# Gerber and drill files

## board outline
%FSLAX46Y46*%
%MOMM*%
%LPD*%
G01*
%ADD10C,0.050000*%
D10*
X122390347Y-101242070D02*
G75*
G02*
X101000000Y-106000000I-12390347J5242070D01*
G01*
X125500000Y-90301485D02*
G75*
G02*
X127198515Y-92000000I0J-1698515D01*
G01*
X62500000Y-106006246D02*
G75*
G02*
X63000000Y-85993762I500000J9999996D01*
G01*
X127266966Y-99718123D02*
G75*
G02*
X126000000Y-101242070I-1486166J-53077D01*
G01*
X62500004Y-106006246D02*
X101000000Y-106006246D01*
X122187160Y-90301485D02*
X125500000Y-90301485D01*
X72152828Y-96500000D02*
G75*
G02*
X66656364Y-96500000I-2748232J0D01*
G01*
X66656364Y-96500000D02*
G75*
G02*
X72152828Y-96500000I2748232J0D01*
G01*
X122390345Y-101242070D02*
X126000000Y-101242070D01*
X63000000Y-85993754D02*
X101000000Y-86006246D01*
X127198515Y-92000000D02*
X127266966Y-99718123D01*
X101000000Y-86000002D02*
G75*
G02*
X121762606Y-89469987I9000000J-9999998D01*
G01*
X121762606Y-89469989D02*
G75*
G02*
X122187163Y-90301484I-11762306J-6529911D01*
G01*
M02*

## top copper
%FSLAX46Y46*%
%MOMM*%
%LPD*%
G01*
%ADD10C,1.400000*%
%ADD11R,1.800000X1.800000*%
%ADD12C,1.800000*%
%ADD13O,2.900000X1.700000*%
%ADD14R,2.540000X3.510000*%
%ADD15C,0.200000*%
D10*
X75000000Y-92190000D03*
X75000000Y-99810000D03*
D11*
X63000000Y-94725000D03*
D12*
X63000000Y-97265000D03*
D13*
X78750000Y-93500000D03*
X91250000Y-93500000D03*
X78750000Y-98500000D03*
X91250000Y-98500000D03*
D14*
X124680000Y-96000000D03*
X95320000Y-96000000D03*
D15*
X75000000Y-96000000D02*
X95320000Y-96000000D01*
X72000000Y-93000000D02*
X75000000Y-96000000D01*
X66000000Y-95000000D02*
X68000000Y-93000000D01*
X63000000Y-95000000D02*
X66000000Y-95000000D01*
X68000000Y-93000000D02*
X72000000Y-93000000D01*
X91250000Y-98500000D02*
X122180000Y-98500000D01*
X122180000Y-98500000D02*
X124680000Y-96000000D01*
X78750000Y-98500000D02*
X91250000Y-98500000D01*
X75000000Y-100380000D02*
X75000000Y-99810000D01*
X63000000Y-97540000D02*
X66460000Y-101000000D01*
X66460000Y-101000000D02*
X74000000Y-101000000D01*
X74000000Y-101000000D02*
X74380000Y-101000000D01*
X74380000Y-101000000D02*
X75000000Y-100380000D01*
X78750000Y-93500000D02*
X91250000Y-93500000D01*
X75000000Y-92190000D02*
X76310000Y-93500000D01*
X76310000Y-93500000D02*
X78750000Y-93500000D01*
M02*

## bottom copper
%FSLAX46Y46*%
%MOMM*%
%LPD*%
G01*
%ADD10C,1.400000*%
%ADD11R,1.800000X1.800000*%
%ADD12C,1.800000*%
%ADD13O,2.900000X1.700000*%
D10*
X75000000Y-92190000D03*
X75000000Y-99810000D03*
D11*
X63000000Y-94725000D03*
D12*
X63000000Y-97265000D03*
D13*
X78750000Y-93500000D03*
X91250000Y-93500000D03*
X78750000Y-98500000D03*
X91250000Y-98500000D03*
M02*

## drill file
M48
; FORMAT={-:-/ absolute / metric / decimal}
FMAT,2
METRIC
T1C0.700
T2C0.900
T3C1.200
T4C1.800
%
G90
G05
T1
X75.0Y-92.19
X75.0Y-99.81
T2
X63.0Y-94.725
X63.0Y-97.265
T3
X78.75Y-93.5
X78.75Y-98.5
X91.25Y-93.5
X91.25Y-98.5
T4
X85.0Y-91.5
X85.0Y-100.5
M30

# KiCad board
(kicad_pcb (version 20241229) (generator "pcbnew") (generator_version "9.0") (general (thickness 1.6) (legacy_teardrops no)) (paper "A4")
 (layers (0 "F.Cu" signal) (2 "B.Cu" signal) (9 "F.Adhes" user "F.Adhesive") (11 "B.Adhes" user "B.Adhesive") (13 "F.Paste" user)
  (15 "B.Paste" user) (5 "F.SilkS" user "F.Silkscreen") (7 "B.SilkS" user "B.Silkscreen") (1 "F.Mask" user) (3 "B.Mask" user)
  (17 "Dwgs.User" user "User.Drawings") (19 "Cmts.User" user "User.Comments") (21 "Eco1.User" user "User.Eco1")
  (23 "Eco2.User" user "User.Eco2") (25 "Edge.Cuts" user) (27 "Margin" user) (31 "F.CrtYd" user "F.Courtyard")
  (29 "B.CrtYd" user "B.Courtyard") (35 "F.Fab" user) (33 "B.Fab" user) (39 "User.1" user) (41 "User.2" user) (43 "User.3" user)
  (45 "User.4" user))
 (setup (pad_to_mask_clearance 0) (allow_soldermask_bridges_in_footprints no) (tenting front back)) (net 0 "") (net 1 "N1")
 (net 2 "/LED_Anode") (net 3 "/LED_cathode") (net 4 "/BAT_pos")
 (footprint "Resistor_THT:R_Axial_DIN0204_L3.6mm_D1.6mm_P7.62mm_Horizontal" (layer "F.Cu") (at 75 92.19 -90)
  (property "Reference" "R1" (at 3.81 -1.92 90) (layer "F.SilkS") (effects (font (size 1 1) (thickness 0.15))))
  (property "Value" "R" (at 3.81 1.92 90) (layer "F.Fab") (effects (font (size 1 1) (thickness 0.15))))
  (pad "1" thru_hole circle (at 0 0 270) (size 1.4 1.4) (drill 0.7) (layers "*.Cu" "*.Mask") (remove_unused_layers no) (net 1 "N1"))
  (pad "2" thru_hole circle (at 7.62 0 270) (size 1.4 1.4) (drill 0.7) (layers "*.Cu" "*.Mask") (remove_unused_layers no)
   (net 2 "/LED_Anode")))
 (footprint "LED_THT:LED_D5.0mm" (layer "F.Cu") (at 63 94.725 -90)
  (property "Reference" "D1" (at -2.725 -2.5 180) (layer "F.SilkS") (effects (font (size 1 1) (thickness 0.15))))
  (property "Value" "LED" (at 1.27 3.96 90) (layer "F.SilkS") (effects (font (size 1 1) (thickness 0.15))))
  (pad "1" thru_hole rect (at 0 0 270) (size 1.8 1.8) (drill 0.9) (layers "*.Cu" "*.Mask") (remove_unused_layers no) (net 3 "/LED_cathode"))
  (pad "2" thru_hole circle (at 2.54 0 270) (size 1.8 1.8) (drill 0.9) (layers "*.Cu" "*.Mask") (remove_unused_layers no)
   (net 2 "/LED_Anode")))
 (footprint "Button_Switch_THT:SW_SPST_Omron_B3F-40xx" (layer "F.Cu") (at 78.75 93.5)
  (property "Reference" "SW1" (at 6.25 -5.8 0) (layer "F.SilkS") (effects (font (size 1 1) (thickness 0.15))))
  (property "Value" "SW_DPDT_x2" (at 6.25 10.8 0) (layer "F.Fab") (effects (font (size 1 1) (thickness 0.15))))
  (pad "" np_thru_hole circle (at 6.25 -2) (size 1.8 1.8) (drill 1.8) (layers "*.Cu" "*.Mask"))
  (pad "" np_thru_hole circle (at 6.25 7) (size 1.8 1.8) (drill 1.8) (layers "*.Cu" "*.Mask"))
  (pad "1" thru_hole oval (at 0 0) (size 2.9 1.7) (drill 1.2) (layers "*.Cu" "*.Mask") (remove_unused_layers no) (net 1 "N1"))
  (pad "1" thru_hole oval (at 12.5 0) (size 2.9 1.7) (drill 1.2) (layers "*.Cu" "*.Mask") (remove_unused_layers no) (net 1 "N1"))
  (pad "2" thru_hole oval (at 0 5) (size 2.9 1.7) (drill 1.2) (layers "*.Cu" "*.Mask") (remove_unused_layers no) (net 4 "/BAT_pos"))
  (pad "2" thru_hole oval (at 12.5 5) (size 2.9 1.7) (drill 1.2) (layers "*.Cu" "*.Mask") (remove_unused_layers no) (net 4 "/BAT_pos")))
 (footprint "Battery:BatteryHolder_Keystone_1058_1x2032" (layer "F.Cu") (at 110 96 180)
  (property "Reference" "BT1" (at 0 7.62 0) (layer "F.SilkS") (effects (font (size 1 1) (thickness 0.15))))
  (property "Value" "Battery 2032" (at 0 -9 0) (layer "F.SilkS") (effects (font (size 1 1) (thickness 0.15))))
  (pad "1" smd rect (at -14.68 0 180) (size 2.54 3.51) (layers "F.Cu" "F.Mask" "F.Paste") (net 4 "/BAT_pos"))
  (pad "2" smd rect (at 14.68 0 180) (size 2.54 3.51) (layers "F.Cu" "F.Mask" "F.Paste") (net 3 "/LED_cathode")))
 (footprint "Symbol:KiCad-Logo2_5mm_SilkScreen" (layer "B.Cu") (at 110 94.5 180)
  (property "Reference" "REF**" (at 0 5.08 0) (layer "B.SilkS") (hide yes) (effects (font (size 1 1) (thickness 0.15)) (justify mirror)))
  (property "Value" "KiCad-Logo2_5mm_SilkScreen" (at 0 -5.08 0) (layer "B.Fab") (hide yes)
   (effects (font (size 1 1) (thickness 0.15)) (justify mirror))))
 (gr_arc (start 122.390347 101.24207) (mid 112.921145 109.132666) (end 101 106) (stroke (width 0.05) (type default)) (locked yes)
  (layer "Edge.Cuts"))
 (gr_arc (start 125.5 90.301485) (mid 126.701031 90.798969) (end 127.198515 92) (stroke (width 0.05) (type default)) (locked yes)
  (layer "Edge.Cuts"))
 (gr_arc (start 62.5 106.006246) (mid 52.990631 95.756168) (end 63 85.993754) (stroke (width 0.05) (type default)) (locked yes)
  (layer "Edge.Cuts"))
 (gr_arc (start 127.266966 99.718123) (mid 126.924335 100.721902) (end 126 101.24207) (stroke (width 0.05) (type default)) (locked yes)
  (layer "Edge.Cuts"))
 (gr_line (start 62.500004 106.006246) (end 101 106.006246) (stroke (width 0.05) (type default)) (locked yes) (layer "Edge.Cuts"))
 (gr_line (start 122.18716 90.301485) (end 125.5 90.301485) (stroke (width 0.05) (type solid)) (locked yes) (layer "Edge.Cuts"))
 (gr_circle (center 69.404596 96.5) (end 71.707372 98) (stroke (width 0.05) (type default)) (fill no) (layer "Edge.Cuts"))
 (gr_line (start 122.390345 101.24207) (end 126 101.24207) (stroke (width 0.05) (type default)) (locked yes) (layer "Edge.Cuts"))
 (gr_line (start 63 85.993754) (end 101 86.006246) (stroke (width 0.05) (type default)) (locked yes) (layer "Edge.Cuts"))
 (gr_line (start 127.198515 92) (end 127.266966 99.718123) (stroke (width 0.05) (type default)) (locked yes) (layer "Edge.Cuts"))
 (gr_arc (start 101 86.000002) (mid 112.217701 82.73042) (end 121.762606 89.469987) (stroke (width 0.05) (type default)) (locked yes)
  (layer "Edge.Cuts"))
 (gr_arc (start 121.762606 89.469989) (mid 121.982098 89.882053) (end 122.18716 90.301485) (stroke (width 0.05) (type default)) (locked yes)
  (layer "Edge.Cuts"))
 (segment (start 75 96) (end 95.32 96) (width 0.2) (layer "F.Cu") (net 3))
 (segment (start 72 93) (end 75 96) (width 0.2) (layer "F.Cu") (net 3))
 (segment (start 66 95) (end 68 93) (width 0.2) (layer "F.Cu") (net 3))
 (segment (start 63 95) (end 66 95) (width 0.2) (layer "F.Cu") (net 3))
 (segment (start 68 93) (end 72 93) (width 0.2) (layer "F.Cu") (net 3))
 (segment (start 91.25 98.5) (end 122.18 98.5) (width 0.2) (layer "F.Cu") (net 4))
 (segment (start 122.18 98.5) (end 124.68 96) (width 0.2) (layer "F.Cu") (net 4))
 (segment (start 78.75 98.5) (end 91.25 98.5) (width 0.2) (layer "F.Cu") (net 4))
 (segment (start 75 100.38) (end 75 99.81) (width 0.2) (layer "F.Cu") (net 2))
 (segment (start 63 97.54) (end 66.46 101) (width 0.2) (layer "F.Cu") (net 2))
 (segment (start 66.46 101) (end 74 101) (width 0.2) (layer "F.Cu") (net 2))
 (segment (start 74 101) (end 74.38 101) (width 0.2) (layer "F.Cu") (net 2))
 (segment (start 74.38 101) (end 75 100.38) (width 0.2) (layer "F.Cu") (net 2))
 (segment (start 78.75 93.5) (end 91.25 93.5) (width 0.2) (layer "F.Cu") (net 1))
 (segment (start 75 92.19) (end 76.31 93.5) (width 0.2) (layer "F.Cu") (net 1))
 (segment (start 76.31 93.5) (end 78.75 93.5) (width 0.2) (layer "F.Cu") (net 1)))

